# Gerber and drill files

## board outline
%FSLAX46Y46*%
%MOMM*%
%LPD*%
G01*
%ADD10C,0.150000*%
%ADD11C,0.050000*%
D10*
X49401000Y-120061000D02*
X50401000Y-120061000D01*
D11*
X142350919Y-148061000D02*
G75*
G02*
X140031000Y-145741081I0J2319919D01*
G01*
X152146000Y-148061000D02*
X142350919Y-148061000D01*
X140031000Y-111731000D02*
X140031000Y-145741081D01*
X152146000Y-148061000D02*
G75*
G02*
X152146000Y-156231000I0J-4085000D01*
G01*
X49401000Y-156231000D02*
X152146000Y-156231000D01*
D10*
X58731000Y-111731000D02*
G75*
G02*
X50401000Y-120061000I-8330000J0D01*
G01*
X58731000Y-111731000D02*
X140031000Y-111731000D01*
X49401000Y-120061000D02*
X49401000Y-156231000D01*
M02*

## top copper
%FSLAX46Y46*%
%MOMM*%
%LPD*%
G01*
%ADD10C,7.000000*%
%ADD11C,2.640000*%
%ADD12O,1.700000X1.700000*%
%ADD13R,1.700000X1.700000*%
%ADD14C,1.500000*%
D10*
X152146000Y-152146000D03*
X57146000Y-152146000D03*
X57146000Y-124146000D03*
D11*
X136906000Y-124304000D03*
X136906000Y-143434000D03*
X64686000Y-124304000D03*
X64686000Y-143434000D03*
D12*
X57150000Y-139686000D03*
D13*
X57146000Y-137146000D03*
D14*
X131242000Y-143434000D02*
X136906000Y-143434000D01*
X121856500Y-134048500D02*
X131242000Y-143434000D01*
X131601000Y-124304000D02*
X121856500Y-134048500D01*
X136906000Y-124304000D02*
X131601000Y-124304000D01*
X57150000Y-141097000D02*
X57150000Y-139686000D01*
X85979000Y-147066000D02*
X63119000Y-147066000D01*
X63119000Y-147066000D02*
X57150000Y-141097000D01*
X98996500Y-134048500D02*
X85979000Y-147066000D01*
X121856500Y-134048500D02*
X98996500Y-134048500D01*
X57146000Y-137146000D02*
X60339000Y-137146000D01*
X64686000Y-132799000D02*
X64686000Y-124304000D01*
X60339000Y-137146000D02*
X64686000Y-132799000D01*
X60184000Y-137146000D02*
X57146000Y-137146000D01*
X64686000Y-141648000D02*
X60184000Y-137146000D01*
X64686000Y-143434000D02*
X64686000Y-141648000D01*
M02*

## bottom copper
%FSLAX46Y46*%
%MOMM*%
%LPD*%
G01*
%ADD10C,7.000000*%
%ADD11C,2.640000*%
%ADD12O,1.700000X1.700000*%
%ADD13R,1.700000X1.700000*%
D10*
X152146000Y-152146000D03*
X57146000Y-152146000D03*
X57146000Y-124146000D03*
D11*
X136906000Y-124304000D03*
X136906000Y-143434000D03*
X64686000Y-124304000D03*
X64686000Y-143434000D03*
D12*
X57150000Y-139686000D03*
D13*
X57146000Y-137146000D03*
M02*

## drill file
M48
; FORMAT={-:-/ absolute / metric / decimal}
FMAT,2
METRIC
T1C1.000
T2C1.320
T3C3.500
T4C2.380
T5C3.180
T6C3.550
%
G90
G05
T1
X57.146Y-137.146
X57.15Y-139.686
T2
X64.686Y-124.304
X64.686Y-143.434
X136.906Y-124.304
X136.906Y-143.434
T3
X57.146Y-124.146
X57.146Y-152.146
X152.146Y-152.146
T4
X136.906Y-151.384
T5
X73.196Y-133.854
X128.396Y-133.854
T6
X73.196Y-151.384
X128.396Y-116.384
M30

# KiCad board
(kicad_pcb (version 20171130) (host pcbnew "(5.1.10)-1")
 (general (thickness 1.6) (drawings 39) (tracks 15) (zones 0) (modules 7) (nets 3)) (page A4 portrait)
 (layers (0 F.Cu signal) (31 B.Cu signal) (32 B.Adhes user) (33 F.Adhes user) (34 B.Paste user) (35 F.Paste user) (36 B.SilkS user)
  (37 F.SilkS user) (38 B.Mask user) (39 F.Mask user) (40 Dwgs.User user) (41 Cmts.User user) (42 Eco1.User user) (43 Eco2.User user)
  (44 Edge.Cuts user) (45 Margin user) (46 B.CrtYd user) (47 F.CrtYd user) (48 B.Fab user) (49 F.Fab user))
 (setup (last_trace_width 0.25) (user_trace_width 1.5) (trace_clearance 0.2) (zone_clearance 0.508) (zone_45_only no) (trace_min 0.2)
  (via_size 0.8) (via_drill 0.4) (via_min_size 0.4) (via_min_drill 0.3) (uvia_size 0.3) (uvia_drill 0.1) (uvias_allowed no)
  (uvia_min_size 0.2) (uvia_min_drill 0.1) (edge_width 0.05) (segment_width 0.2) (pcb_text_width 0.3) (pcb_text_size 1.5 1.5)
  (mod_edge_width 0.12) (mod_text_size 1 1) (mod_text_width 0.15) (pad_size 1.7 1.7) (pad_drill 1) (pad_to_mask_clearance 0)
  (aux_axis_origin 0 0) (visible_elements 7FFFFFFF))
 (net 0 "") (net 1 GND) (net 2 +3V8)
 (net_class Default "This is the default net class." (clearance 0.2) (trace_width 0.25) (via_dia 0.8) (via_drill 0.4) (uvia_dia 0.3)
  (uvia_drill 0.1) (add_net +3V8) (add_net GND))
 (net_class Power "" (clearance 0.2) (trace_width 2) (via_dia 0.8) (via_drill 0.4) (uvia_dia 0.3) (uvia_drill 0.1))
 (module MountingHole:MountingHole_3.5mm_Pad (layer F.Cu) (at 152.146 152.146)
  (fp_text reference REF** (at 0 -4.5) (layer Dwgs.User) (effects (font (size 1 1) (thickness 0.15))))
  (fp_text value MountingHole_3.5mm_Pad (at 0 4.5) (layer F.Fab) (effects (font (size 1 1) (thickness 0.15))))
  (pad 1 thru_hole circle (at 0 0) (size 7 7) (drill 3.5) (layers *.Cu *.Mask)))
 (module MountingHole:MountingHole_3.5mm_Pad (layer F.Cu) (at 57.146 152.146)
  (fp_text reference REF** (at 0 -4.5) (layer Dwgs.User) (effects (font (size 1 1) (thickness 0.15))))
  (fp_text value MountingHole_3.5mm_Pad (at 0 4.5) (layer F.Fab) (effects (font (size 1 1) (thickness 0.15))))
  (pad 1 thru_hole circle (at 0 0) (size 7 7) (drill 3.5) (layers *.Cu *.Mask)))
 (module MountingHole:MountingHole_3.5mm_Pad (layer F.Cu) (at 57.146 124.146)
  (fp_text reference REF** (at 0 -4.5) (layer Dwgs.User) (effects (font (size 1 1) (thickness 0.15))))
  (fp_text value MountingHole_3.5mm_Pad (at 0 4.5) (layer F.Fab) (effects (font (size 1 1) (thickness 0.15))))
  (pad 1 thru_hole circle (at 0 0) (size 7 7) (drill 3.5) (layers *.Cu *.Mask)))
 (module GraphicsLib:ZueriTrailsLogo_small (layer F.Cu) (at 100.33 124.206)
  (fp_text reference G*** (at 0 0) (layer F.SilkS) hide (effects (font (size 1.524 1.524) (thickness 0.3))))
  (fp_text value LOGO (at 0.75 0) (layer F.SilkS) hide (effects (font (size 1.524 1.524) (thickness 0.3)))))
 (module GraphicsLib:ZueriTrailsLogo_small (layer F.Cu) (at 100.33 143.51)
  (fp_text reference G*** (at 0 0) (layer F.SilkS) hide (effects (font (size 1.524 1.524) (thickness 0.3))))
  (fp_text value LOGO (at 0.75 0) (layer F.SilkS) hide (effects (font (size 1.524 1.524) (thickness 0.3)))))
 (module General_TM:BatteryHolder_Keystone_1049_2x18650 (layer F.Cu) (at 64.686 151.384)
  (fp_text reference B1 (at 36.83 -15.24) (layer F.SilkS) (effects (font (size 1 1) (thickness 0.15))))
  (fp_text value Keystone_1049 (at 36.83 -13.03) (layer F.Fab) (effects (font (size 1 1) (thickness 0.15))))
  (pad "" np_thru_hole circle (at 72.22 0) (size 2.38 2.38) (drill 2.38) (layers *.Cu *.Mask))
  (pad "" np_thru_hole circle (at 63.71 -35) (size 3.55 3.55) (drill 3.55) (layers *.Cu *.Mask))
  (pad "" np_thru_hole circle (at 8.51 0) (size 3.55 3.55) (drill 3.55) (layers *.Cu *.Mask))
  (pad "" np_thru_hole circle (at 63.71 -17.53) (size 3.18 3.18) (drill 3.18) (layers *.Cu *.Mask))
  (pad "" np_thru_hole circle (at 8.51 -17.53) (size 3.18 3.18) (drill 3.18) (layers *.Cu *.Mask))
  (pad 4 thru_hole circle (at 72.22 -27.08) (size 2.64 2.64) (drill 1.32) (layers *.Cu *.Mask) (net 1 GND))
  (pad 2 thru_hole circle (at 72.22 -7.95) (size 2.64 2.64) (drill 1.32) (layers *.Cu *.Mask) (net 1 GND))
  (pad 3 thru_hole circle (at 0 -27.08) (size 2.64 2.64) (drill 1.32) (layers *.Cu *.Mask) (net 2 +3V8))
  (pad 1 thru_hole circle (at 0 -7.95) (size 2.64 2.64) (drill 1.32) (layers *.Cu *.Mask) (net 2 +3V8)))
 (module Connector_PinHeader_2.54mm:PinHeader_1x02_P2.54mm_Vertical (layer F.Cu) (at 57.15 137.146)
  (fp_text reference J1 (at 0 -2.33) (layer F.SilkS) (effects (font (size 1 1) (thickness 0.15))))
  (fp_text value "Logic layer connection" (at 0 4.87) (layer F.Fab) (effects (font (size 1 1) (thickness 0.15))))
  (pad 2 thru_hole oval (at 0 2.54) (size 1.7 1.7) (drill 1) (layers *.Cu *.Mask) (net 1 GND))
  (pad 1 thru_hole rect (at -0.004 0) (size 1.7 1.7) (drill 1) (layers *.Cu *.Mask) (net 2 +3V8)))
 (gr_line (start 49.401 120.061) (end 50.401 120.061) (layer Edge.Cuts) (width 0.15))
 (gr_arc (start 142.350919 145.741081) (end 140.031 145.741081) (angle -90) (layer Edge.Cuts) (width 0.05))
 (gr_line (start 152.146 148.061) (end 142.350919 148.061) (layer Edge.Cuts) (width 0.05))
 (gr_line (start 140.031 111.731) (end 140.031 145.741081) (layer Edge.Cuts) (width 0.05))
 (gr_arc (start 152.146 152.146) (end 152.146 156.231) (angle -180) (layer Edge.Cuts) (width 0.05))
 (gr_line (start 49.401 156.231) (end 152.146 156.231) (layer Edge.Cuts) (width 0.05))
 (gr_arc (start 50.401 111.731) (end 58.731 111.731) (angle 90) (layer Edge.Cuts) (width 0.15))
 (gr_line (start 58.731 111.731) (end 140.031 111.731) (layer Edge.Cuts) (width 0.15))
 (gr_line (start 49.401 120.061) (end 49.401 156.231) (layer Edge.Cuts) (width 0.15))
 (segment (start 131.242 143.434) (end 136.906 143.434) (width 1.5) (layer F.Cu) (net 1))
 (segment (start 121.8565 134.0485) (end 131.242 143.434) (width 1.5) (layer F.Cu) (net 1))
 (segment (start 131.601 124.304) (end 121.8565 134.0485) (width 1.5) (layer F.Cu) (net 1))
 (segment (start 136.906 124.304) (end 131.601 124.304) (width 1.5) (layer F.Cu) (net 1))
 (segment (start 57.15 141.097) (end 57.15 139.686) (width 1.5) (layer F.Cu) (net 1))
 (segment (start 85.979 147.066) (end 63.119 147.066) (width 1.5) (layer F.Cu) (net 1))
 (segment (start 63.119 147.066) (end 57.15 141.097) (width 1.5) (layer F.Cu) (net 1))
 (segment (start 98.9965 134.0485) (end 85.979 147.066) (width 1.5) (layer F.Cu) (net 1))
 (segment (start 121.8565 134.0485) (end 98.9965 134.0485) (width 1.5) (layer F.Cu) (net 1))
 (segment (start 57.146 137.146) (end 60.339 137.146) (width 1.5) (layer F.Cu) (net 2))
 (segment (start 64.686 132.799) (end 64.686 124.304) (width 1.5) (layer F.Cu) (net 2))
 (segment (start 60.339 137.146) (end 64.686 132.799) (width 1.5) (layer F.Cu) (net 2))
 (segment (start 60.184 137.146) (end 57.146 137.146) (width 1.5) (layer F.Cu) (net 2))
 (segment (start 64.686 141.648) (end 60.184 137.146) (width 1.5) (layer F.Cu) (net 2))
 (segment (start 64.686 143.434) (end 64.686 141.648) (width 1.5) (layer F.Cu) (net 2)))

